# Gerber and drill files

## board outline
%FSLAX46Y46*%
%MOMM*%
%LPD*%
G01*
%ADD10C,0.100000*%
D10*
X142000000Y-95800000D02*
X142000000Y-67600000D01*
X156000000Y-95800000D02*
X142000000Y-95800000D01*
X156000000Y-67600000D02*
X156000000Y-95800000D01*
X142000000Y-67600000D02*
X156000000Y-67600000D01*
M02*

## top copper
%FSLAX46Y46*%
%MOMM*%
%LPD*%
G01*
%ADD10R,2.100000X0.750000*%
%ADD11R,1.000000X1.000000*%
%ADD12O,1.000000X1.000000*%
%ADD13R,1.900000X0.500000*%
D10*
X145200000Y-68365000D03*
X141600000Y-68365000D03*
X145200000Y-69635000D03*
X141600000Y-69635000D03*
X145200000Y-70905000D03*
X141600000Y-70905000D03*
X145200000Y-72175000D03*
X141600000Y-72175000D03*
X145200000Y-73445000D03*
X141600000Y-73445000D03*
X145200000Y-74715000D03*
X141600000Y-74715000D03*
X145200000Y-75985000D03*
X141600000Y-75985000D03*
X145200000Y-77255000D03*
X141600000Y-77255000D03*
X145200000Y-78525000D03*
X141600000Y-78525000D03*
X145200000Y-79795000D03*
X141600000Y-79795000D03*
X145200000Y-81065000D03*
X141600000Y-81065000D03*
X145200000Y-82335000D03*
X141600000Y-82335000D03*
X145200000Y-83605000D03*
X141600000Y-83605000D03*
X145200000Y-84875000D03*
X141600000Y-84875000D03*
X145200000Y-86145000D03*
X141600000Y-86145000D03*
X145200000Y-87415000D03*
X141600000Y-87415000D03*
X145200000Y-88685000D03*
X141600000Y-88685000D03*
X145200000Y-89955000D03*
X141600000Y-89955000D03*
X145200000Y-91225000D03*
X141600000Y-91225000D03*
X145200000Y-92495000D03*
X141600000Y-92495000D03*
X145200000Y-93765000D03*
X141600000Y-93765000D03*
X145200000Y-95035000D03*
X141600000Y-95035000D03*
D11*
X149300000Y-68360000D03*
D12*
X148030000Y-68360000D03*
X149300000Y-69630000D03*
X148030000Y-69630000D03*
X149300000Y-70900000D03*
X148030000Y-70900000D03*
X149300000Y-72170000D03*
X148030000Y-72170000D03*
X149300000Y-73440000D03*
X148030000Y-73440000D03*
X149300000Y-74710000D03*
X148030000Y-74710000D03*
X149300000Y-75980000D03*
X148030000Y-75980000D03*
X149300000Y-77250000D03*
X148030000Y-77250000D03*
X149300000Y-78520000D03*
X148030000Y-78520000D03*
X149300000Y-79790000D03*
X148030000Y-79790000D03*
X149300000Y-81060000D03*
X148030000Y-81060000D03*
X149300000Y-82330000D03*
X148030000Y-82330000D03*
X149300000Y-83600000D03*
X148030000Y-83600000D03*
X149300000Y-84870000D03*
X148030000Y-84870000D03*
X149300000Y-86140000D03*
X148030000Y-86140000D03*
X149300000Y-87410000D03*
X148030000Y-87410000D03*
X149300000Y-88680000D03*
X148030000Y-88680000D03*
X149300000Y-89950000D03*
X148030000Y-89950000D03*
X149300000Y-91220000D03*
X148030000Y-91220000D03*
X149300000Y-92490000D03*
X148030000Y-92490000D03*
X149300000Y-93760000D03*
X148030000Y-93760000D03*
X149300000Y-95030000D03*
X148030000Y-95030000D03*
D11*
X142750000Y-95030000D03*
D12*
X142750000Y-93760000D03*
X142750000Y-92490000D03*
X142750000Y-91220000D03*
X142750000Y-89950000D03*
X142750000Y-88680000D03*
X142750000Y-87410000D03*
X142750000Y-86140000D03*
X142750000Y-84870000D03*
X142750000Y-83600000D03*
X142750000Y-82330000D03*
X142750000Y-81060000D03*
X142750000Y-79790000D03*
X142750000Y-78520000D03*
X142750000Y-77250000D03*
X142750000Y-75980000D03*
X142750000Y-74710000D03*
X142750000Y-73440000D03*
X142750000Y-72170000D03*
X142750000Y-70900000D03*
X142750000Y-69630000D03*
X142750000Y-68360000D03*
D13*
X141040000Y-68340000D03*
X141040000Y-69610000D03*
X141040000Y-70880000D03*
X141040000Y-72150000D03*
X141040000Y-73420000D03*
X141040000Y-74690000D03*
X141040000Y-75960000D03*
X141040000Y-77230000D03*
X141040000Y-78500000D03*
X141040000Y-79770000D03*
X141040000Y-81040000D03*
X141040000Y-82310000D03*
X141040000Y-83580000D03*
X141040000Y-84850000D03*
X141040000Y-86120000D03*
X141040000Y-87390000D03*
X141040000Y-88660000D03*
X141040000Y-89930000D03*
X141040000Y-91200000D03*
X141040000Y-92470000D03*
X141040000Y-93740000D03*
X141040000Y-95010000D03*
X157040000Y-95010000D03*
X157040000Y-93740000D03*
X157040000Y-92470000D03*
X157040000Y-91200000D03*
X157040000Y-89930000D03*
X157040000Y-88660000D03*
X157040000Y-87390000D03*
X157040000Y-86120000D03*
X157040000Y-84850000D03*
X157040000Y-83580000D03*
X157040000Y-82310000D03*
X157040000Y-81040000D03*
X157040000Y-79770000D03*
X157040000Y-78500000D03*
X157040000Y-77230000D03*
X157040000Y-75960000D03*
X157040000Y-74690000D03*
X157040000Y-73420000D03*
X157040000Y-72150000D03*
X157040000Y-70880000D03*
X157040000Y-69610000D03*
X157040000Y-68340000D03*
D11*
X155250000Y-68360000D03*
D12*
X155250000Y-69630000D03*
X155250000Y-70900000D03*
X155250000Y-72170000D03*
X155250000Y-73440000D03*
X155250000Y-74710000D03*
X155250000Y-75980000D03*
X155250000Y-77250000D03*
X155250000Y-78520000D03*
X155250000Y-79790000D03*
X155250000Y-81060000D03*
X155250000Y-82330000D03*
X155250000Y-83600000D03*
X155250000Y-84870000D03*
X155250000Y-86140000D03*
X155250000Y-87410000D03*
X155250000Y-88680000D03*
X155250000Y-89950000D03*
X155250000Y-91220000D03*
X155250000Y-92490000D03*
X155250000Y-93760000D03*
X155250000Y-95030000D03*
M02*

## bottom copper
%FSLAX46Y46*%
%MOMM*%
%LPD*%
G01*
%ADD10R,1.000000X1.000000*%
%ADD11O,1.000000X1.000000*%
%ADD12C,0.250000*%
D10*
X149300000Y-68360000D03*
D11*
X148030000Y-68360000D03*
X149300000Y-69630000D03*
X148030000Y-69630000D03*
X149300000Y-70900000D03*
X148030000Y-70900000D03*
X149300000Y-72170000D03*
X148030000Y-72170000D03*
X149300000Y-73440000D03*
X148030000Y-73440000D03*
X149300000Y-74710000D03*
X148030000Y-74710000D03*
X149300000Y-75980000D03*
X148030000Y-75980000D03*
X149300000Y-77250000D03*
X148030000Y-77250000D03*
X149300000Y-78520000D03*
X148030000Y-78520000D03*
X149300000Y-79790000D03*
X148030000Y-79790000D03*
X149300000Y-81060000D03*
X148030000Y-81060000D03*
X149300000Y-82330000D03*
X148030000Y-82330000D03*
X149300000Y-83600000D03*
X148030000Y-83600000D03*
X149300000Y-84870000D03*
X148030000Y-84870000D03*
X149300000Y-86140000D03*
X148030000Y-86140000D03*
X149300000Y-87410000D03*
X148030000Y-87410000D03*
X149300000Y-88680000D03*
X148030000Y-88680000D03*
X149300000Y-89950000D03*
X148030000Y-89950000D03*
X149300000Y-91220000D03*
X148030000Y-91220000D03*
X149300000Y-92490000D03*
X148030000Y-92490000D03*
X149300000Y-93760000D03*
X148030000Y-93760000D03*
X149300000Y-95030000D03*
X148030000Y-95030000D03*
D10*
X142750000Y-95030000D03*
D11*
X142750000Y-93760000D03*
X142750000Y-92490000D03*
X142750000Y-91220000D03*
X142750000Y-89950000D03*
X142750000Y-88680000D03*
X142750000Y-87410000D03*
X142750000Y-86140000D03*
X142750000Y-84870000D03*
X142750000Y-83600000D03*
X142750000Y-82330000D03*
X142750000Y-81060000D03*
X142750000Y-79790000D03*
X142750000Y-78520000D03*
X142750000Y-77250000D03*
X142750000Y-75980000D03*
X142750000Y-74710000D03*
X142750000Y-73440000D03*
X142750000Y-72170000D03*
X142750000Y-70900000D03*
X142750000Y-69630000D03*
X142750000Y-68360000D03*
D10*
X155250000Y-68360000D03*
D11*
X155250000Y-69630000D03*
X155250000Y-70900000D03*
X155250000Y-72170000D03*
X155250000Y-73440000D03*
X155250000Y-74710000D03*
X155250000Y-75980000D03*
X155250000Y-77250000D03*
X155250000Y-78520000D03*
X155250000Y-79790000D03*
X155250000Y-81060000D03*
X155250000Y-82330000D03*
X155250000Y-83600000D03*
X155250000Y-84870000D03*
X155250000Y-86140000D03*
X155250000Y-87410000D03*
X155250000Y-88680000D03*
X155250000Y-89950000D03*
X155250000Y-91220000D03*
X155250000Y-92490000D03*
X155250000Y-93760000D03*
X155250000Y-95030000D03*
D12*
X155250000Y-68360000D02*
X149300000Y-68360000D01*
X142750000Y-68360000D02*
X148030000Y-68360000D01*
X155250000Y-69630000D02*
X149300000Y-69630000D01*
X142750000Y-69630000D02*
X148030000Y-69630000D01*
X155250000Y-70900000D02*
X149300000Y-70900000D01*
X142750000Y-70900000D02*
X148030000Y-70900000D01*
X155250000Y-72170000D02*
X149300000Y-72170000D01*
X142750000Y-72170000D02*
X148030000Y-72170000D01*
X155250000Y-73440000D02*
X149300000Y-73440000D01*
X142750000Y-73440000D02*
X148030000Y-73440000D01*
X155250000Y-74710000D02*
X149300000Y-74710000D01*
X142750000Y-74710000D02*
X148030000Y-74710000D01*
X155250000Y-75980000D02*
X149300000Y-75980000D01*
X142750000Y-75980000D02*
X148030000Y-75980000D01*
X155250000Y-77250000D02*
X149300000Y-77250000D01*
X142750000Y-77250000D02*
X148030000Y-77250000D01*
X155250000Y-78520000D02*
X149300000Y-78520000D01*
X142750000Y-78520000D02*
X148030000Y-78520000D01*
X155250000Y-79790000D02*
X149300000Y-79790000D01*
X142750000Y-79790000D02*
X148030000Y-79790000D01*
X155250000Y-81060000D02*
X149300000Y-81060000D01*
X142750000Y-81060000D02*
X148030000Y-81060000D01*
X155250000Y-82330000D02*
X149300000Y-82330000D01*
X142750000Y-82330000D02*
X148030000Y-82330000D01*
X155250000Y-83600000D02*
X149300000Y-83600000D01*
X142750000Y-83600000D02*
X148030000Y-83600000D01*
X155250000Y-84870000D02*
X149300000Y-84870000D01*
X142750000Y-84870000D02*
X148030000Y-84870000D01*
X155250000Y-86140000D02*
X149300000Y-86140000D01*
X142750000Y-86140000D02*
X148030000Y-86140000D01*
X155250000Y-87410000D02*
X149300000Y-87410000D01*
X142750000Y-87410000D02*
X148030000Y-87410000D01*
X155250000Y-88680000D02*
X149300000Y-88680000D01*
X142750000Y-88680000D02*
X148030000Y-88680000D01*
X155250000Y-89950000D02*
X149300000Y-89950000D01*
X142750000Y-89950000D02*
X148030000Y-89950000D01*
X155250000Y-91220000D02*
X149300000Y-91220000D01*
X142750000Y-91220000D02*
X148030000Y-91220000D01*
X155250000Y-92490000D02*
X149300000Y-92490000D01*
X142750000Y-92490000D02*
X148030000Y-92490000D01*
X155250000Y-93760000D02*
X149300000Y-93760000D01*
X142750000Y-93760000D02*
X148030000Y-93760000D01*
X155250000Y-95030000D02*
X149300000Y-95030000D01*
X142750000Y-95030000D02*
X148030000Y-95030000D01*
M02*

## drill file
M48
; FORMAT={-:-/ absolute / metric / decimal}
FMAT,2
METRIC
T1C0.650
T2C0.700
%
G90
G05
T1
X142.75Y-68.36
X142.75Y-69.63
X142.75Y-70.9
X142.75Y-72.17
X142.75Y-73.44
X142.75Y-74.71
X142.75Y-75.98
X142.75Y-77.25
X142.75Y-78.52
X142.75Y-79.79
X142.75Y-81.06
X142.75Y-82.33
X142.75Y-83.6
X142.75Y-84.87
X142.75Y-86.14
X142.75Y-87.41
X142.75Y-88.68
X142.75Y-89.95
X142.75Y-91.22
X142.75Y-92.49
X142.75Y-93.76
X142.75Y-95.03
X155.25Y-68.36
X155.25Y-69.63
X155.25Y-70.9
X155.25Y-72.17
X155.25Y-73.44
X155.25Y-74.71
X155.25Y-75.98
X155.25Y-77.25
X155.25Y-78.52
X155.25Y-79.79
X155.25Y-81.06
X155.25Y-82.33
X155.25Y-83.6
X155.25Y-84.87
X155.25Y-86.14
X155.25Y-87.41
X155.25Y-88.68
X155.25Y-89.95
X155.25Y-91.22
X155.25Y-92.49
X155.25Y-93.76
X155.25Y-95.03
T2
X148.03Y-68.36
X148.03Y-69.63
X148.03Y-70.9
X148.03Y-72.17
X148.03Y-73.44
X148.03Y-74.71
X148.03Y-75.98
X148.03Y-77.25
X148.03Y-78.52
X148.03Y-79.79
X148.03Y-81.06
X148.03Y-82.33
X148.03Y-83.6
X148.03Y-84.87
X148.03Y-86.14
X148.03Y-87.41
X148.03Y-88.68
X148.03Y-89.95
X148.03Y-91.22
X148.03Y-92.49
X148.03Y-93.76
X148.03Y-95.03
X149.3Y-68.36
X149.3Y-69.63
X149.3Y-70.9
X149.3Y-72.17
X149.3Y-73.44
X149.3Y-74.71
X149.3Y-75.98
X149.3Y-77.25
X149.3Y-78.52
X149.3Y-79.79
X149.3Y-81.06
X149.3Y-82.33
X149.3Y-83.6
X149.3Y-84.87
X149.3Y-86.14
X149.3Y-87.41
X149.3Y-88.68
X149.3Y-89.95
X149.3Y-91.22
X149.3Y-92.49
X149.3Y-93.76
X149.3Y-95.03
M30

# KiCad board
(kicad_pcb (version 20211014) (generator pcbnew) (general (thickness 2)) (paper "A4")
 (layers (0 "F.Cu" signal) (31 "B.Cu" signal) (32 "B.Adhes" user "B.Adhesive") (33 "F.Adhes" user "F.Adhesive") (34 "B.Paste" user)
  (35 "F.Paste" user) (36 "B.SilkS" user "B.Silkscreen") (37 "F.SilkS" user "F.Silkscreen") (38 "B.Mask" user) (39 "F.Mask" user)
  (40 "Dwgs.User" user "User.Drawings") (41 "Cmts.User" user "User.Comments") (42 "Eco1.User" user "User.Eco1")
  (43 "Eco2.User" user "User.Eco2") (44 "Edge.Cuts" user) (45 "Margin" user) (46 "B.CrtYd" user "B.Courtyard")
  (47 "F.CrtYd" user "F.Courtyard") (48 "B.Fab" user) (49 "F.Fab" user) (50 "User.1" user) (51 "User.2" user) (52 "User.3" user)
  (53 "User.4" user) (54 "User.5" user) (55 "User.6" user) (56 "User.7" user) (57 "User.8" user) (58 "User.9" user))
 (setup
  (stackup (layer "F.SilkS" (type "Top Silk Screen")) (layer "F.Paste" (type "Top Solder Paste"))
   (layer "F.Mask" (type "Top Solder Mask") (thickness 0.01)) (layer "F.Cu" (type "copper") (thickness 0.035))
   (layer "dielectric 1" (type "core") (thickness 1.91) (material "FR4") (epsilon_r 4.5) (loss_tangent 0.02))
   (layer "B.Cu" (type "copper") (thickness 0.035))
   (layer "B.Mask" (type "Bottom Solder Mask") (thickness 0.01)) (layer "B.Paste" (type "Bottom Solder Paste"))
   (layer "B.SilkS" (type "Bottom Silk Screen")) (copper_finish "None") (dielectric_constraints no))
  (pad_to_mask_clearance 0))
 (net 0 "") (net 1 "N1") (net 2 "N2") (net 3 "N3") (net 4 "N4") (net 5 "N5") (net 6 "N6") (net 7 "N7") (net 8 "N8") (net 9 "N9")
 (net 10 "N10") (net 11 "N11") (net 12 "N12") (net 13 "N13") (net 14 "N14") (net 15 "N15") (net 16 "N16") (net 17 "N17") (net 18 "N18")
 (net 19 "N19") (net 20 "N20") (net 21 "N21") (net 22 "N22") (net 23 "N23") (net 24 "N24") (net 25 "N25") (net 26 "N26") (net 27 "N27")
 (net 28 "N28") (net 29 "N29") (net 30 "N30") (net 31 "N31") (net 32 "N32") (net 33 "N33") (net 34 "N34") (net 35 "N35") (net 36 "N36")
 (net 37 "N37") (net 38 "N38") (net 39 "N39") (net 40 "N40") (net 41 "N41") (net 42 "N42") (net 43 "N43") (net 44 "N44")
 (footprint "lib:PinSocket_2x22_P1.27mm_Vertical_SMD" (layer "F.Cu") (at 143.4 81.7)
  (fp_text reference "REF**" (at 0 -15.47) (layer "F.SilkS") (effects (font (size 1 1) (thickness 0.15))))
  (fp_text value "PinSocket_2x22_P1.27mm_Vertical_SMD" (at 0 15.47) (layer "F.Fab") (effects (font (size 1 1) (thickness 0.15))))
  (pad "1" smd rect (at 1.8 -13.335) (size 2.1 0.75) (layers "F.Cu" "F.Paste" "F.Mask"))
  (pad "2" smd rect (at -1.8 -13.335) (size 2.1 0.75) (layers "F.Cu" "F.Paste" "F.Mask"))
  (pad "3" smd rect (at 1.8 -12.065) (size 2.1 0.75) (layers "F.Cu" "F.Paste" "F.Mask"))
  (pad "4" smd rect (at -1.8 -12.065) (size 2.1 0.75) (layers "F.Cu" "F.Paste" "F.Mask"))
  (pad "5" smd rect (at 1.8 -10.795) (size 2.1 0.75) (layers "F.Cu" "F.Paste" "F.Mask"))
  (pad "6" smd rect (at -1.8 -10.795) (size 2.1 0.75) (layers "F.Cu" "F.Paste" "F.Mask"))
  (pad "7" smd rect (at 1.8 -9.525) (size 2.1 0.75) (layers "F.Cu" "F.Paste" "F.Mask"))
  (pad "8" smd rect (at -1.8 -9.525) (size 2.1 0.75) (layers "F.Cu" "F.Paste" "F.Mask"))
  (pad "9" smd rect (at 1.8 -8.255) (size 2.1 0.75) (layers "F.Cu" "F.Paste" "F.Mask"))
  (pad "10" smd rect (at -1.8 -8.255) (size 2.1 0.75) (layers "F.Cu" "F.Paste" "F.Mask"))
  (pad "11" smd rect (at 1.8 -6.985) (size 2.1 0.75) (layers "F.Cu" "F.Paste" "F.Mask"))
  (pad "12" smd rect (at -1.8 -6.985) (size 2.1 0.75) (layers "F.Cu" "F.Paste" "F.Mask"))
  (pad "13" smd rect (at 1.8 -5.715) (size 2.1 0.75) (layers "F.Cu" "F.Paste" "F.Mask"))
  (pad "14" smd rect (at -1.8 -5.715) (size 2.1 0.75) (layers "F.Cu" "F.Paste" "F.Mask"))
  (pad "15" smd rect (at 1.8 -4.445) (size 2.1 0.75) (layers "F.Cu" "F.Paste" "F.Mask"))
  (pad "16" smd rect (at -1.8 -4.445) (size 2.1 0.75) (layers "F.Cu" "F.Paste" "F.Mask"))
  (pad "17" smd rect (at 1.8 -3.175) (size 2.1 0.75) (layers "F.Cu" "F.Paste" "F.Mask"))
  (pad "18" smd rect (at -1.8 -3.175) (size 2.1 0.75) (layers "F.Cu" "F.Paste" "F.Mask"))
  (pad "19" smd rect (at 1.8 -1.905) (size 2.1 0.75) (layers "F.Cu" "F.Paste" "F.Mask"))
  (pad "20" smd rect (at -1.8 -1.905) (size 2.1 0.75) (layers "F.Cu" "F.Paste" "F.Mask"))
  (pad "21" smd rect (at 1.8 -0.635) (size 2.1 0.75) (layers "F.Cu" "F.Paste" "F.Mask"))
  (pad "22" smd rect (at -1.8 -0.635) (size 2.1 0.75) (layers "F.Cu" "F.Paste" "F.Mask"))
  (pad "23" smd rect (at 1.8 0.635) (size 2.1 0.75) (layers "F.Cu" "F.Paste" "F.Mask"))
  (pad "24" smd rect (at -1.8 0.635) (size 2.1 0.75) (layers "F.Cu" "F.Paste" "F.Mask"))
  (pad "25" smd rect (at 1.8 1.905) (size 2.1 0.75) (layers "F.Cu" "F.Paste" "F.Mask"))
  (pad "26" smd rect (at -1.8 1.905) (size 2.1 0.75) (layers "F.Cu" "F.Paste" "F.Mask"))
  (pad "27" smd rect (at 1.8 3.175) (size 2.1 0.75) (layers "F.Cu" "F.Paste" "F.Mask"))
  (pad "28" smd rect (at -1.8 3.175) (size 2.1 0.75) (layers "F.Cu" "F.Paste" "F.Mask"))
  (pad "29" smd rect (at 1.8 4.445) (size 2.1 0.75) (layers "F.Cu" "F.Paste" "F.Mask"))
  (pad "30" smd rect (at -1.8 4.445) (size 2.1 0.75) (layers "F.Cu" "F.Paste" "F.Mask"))
  (pad "31" smd rect (at 1.8 5.715) (size 2.1 0.75) (layers "F.Cu" "F.Paste" "F.Mask"))
  (pad "32" smd rect (at -1.8 5.715) (size 2.1 0.75) (layers "F.Cu" "F.Paste" "F.Mask"))
  (pad "33" smd rect (at 1.8 6.985) (size 2.1 0.75) (layers "F.Cu" "F.Paste" "F.Mask"))
  (pad "34" smd rect (at -1.8 6.985) (size 2.1 0.75) (layers "F.Cu" "F.Paste" "F.Mask"))
  (pad "35" smd rect (at 1.8 8.255) (size 2.1 0.75) (layers "F.Cu" "F.Paste" "F.Mask"))
  (pad "36" smd rect (at -1.8 8.255) (size 2.1 0.75) (layers "F.Cu" "F.Paste" "F.Mask"))
  (pad "37" smd rect (at 1.8 9.525) (size 2.1 0.75) (layers "F.Cu" "F.Paste" "F.Mask"))
  (pad "38" smd rect (at -1.8 9.525) (size 2.1 0.75) (layers "F.Cu" "F.Paste" "F.Mask"))
  (pad "39" smd rect (at 1.8 10.795) (size 2.1 0.75) (layers "F.Cu" "F.Paste" "F.Mask"))
  (pad "40" smd rect (at -1.8 10.795) (size 2.1 0.75) (layers "F.Cu" "F.Paste" "F.Mask"))
  (pad "41" smd rect (at 1.8 12.065) (size 2.1 0.75) (layers "F.Cu" "F.Paste" "F.Mask"))
  (pad "42" smd rect (at -1.8 12.065) (size 2.1 0.75) (layers "F.Cu" "F.Paste" "F.Mask"))
  (pad "43" smd rect (at 1.8 13.335) (size 2.1 0.75) (layers "F.Cu" "F.Paste" "F.Mask"))
  (pad "44" smd rect (at -1.8 13.335) (size 2.1 0.75) (layers "F.Cu" "F.Paste" "F.Mask")))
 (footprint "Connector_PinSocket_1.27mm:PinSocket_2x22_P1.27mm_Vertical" (layer "F.Cu") (at 149.3 68.36)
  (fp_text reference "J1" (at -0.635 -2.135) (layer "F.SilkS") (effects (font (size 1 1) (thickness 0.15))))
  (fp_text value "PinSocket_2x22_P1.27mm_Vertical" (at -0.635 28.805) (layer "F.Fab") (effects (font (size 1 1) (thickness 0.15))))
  (pad "1" thru_hole rect (at 0 0) (size 1 1) (drill 0.7) (layers *.Cu *.Mask) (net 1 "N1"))
  (pad "2" thru_hole oval (at -1.27 0) (size 1 1) (drill 0.7) (layers *.Cu *.Mask) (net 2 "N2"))
  (pad "3" thru_hole oval (at 0 1.27) (size 1 1) (drill 0.7) (layers *.Cu *.Mask) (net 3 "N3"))
  (pad "4" thru_hole oval (at -1.27 1.27) (size 1 1) (drill 0.7) (layers *.Cu *.Mask) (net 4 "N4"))
  (pad "5" thru_hole oval (at 0 2.54) (size 1 1) (drill 0.7) (layers *.Cu *.Mask) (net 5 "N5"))
  (pad "6" thru_hole oval (at -1.27 2.54) (size 1 1) (drill 0.7) (layers *.Cu *.Mask) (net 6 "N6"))
  (pad "7" thru_hole oval (at 0 3.81) (size 1 1) (drill 0.7) (layers *.Cu *.Mask) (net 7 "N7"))
  (pad "8" thru_hole oval (at -1.27 3.81) (size 1 1) (drill 0.7) (layers *.Cu *.Mask) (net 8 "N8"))
  (pad "9" thru_hole oval (at 0 5.08) (size 1 1) (drill 0.7) (layers *.Cu *.Mask) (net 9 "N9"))
  (pad "10" thru_hole oval (at -1.27 5.08) (size 1 1) (drill 0.7) (layers *.Cu *.Mask) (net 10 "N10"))
  (pad "11" thru_hole oval (at 0 6.35) (size 1 1) (drill 0.7) (layers *.Cu *.Mask) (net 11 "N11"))
  (pad "12" thru_hole oval (at -1.27 6.35) (size 1 1) (drill 0.7) (layers *.Cu *.Mask) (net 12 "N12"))
  (pad "13" thru_hole oval (at 0 7.62) (size 1 1) (drill 0.7) (layers *.Cu *.Mask) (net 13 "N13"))
  (pad "14" thru_hole oval (at -1.27 7.62) (size 1 1) (drill 0.7) (layers *.Cu *.Mask) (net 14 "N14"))
  (pad "15" thru_hole oval (at 0 8.89) (size 1 1) (drill 0.7) (layers *.Cu *.Mask) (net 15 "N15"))
  (pad "16" thru_hole oval (at -1.27 8.89) (size 1 1) (drill 0.7) (layers *.Cu *.Mask) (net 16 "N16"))
  (pad "17" thru_hole oval (at 0 10.16) (size 1 1) (drill 0.7) (layers *.Cu *.Mask) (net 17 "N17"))
  (pad "18" thru_hole oval (at -1.27 10.16) (size 1 1) (drill 0.7) (layers *.Cu *.Mask) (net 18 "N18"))
  (pad "19" thru_hole oval (at 0 11.43) (size 1 1) (drill 0.7) (layers *.Cu *.Mask) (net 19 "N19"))
  (pad "20" thru_hole oval (at -1.27 11.43) (size 1 1) (drill 0.7) (layers *.Cu *.Mask) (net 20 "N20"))
  (pad "21" thru_hole oval (at 0 12.7) (size 1 1) (drill 0.7) (layers *.Cu *.Mask) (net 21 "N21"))
  (pad "22" thru_hole oval (at -1.27 12.7) (size 1 1) (drill 0.7) (layers *.Cu *.Mask) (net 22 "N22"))
  (pad "23" thru_hole oval (at 0 13.97) (size 1 1) (drill 0.7) (layers *.Cu *.Mask) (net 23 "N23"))
  (pad "24" thru_hole oval (at -1.27 13.97) (size 1 1) (drill 0.7) (layers *.Cu *.Mask) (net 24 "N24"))
  (pad "25" thru_hole oval (at 0 15.24) (size 1 1) (drill 0.7) (layers *.Cu *.Mask) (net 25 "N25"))
  (pad "26" thru_hole oval (at -1.27 15.24) (size 1 1) (drill 0.7) (layers *.Cu *.Mask) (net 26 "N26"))
  (pad "27" thru_hole oval (at 0 16.51) (size 1 1) (drill 0.7) (layers *.Cu *.Mask) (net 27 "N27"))
  (pad "28" thru_hole oval (at -1.27 16.51) (size 1 1) (drill 0.7) (layers *.Cu *.Mask) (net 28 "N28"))
  (pad "29" thru_hole oval (at 0 17.78) (size 1 1) (drill 0.7) (layers *.Cu *.Mask) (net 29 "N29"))
  (pad "30" thru_hole oval (at -1.27 17.78) (size 1 1) (drill 0.7) (layers *.Cu *.Mask) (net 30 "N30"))
  (pad "31" thru_hole oval (at 0 19.05) (size 1 1) (drill 0.7) (layers *.Cu *.Mask) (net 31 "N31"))
  (pad "32" thru_hole oval (at -1.27 19.05) (size 1 1) (drill 0.7) (layers *.Cu *.Mask) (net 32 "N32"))
  (pad "33" thru_hole oval (at 0 20.32) (size 1 1) (drill 0.7) (layers *.Cu *.Mask) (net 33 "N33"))
  (pad "34" thru_hole oval (at -1.27 20.32) (size 1 1) (drill 0.7) (layers *.Cu *.Mask) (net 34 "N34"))
  (pad "35" thru_hole oval (at 0 21.59) (size 1 1) (drill 0.7) (layers *.Cu *.Mask) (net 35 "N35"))
  (pad "36" thru_hole oval (at -1.27 21.59) (size 1 1) (drill 0.7) (layers *.Cu *.Mask) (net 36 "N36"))
  (pad "37" thru_hole oval (at 0 22.86) (size 1 1) (drill 0.7) (layers *.Cu *.Mask) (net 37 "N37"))
  (pad "38" thru_hole oval (at -1.27 22.86) (size 1 1) (drill 0.7) (layers *.Cu *.Mask) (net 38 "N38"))
  (pad "39" thru_hole oval (at 0 24.13) (size 1 1) (drill 0.7) (layers *.Cu *.Mask) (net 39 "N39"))
  (pad "40" thru_hole oval (at -1.27 24.13) (size 1 1) (drill 0.7) (layers *.Cu *.Mask) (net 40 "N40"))
  (pad "41" thru_hole oval (at 0 25.4) (size 1 1) (drill 0.7) (layers *.Cu *.Mask) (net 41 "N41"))
  (pad "42" thru_hole oval (at -1.27 25.4) (size 1 1) (drill 0.7) (layers *.Cu *.Mask) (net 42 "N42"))
  (pad "43" thru_hole oval (at 0 26.67) (size 1 1) (drill 0.7) (layers *.Cu *.Mask) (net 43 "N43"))
  (pad "44" thru_hole oval (at -1.27 26.67) (size 1 1) (drill 0.7) (layers *.Cu *.Mask) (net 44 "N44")))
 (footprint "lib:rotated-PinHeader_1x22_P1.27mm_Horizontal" (layer "F.Cu") (at 142.75 95.03 180)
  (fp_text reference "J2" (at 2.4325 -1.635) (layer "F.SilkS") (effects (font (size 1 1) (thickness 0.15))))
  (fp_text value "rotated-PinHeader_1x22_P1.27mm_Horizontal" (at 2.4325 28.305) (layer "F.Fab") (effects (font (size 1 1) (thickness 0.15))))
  (pad "1" thru_hole rect (at 0 0 180) (size 1 1) (drill 0.65) (layers *.Cu *.Mask) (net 44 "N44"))
  (pad "2" thru_hole oval (at 0 1.27 180) (size 1 1) (drill 0.65) (layers *.Cu *.Mask) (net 42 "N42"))
  (pad "3" thru_hole oval (at 0 2.54 180) (size 1 1) (drill 0.65) (layers *.Cu *.Mask) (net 40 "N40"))
  (pad "4" thru_hole oval (at 0 3.81 180) (size 1 1) (drill 0.65) (layers *.Cu *.Mask) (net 38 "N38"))
  (pad "5" thru_hole oval (at 0 5.08 180) (size 1 1) (drill 0.65) (layers *.Cu *.Mask) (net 36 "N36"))
  (pad "6" thru_hole oval (at 0 6.35 180) (size 1 1) (drill 0.65) (layers *.Cu *.Mask) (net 34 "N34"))
  (pad "7" thru_hole oval (at 0 7.62 180) (size 1 1) (drill 0.65) (layers *.Cu *.Mask) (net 32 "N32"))
  (pad "8" thru_hole oval (at 0 8.89 180) (size 1 1) (drill 0.65) (layers *.Cu *.Mask) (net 30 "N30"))
  (pad "9" thru_hole oval (at 0 10.16 180) (size 1 1) (drill 0.65) (layers *.Cu *.Mask) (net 28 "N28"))
  (pad "10" thru_hole oval (at 0 11.43 180) (size 1 1) (drill 0.65) (layers *.Cu *.Mask) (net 26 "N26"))
  (pad "11" thru_hole oval (at 0 12.7 180) (size 1 1) (drill 0.65) (layers *.Cu *.Mask) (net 24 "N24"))
  (pad "12" thru_hole oval (at 0 13.97 180) (size 1 1) (drill 0.65) (layers *.Cu *.Mask) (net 22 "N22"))
  (pad "13" thru_hole oval (at 0 15.24 180) (size 1 1) (drill 0.65) (layers *.Cu *.Mask) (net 20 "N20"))
  (pad "14" thru_hole oval (at 0 16.51 180) (size 1 1) (drill 0.65) (layers *.Cu *.Mask) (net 18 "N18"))
  (pad "15" thru_hole oval (at 0 17.78 180) (size 1 1) (drill 0.65) (layers *.Cu *.Mask) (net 16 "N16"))
  (pad "16" thru_hole oval (at 0 19.05 180) (size 1 1) (drill 0.65) (layers *.Cu *.Mask) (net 14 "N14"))
  (pad "17" thru_hole oval (at 0 20.32 180) (size 1 1) (drill 0.65) (layers *.Cu *.Mask) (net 12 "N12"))
  (pad "18" thru_hole oval (at 0 21.59 180) (size 1 1) (drill 0.65) (layers *.Cu *.Mask) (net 10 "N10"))
  (pad "19" thru_hole oval (at 0 22.86 180) (size 1 1) (drill 0.65) (layers *.Cu *.Mask) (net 8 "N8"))
  (pad "20" thru_hole oval (at 0 24.13 180) (size 1 1) (drill 0.65) (layers *.Cu *.Mask) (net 6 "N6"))
  (pad "21" thru_hole oval (at 0 25.4 180) (size 1 1) (drill 0.65) (layers *.Cu *.Mask) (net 4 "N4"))
  (pad "22" thru_hole oval (at 0 26.67 180) (size 1 1) (drill 0.65) (layers *.Cu *.Mask) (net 2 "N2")))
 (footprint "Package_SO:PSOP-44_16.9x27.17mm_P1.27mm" (layer "F.Cu") (at 149.04 81.675)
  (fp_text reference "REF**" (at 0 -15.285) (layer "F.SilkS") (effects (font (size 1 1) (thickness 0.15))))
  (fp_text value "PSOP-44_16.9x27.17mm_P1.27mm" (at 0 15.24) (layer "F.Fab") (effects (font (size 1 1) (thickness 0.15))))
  (pad "1" smd rect (at -8 -13.335 270) (size 0.5 1.9) (layers "F.Cu" "F.Paste" "F.Mask"))
  (pad "2" smd rect (at -8 -12.065 270) (size 0.5 1.9) (layers "F.Cu" "F.Paste" "F.Mask"))
  (pad "3" smd rect (at -8 -10.795 270) (size 0.5 1.9) (layers "F.Cu" "F.Paste" "F.Mask"))
  (pad "4" smd rect (at -8 -9.525 270) (size 0.5 1.9) (layers "F.Cu" "F.Paste" "F.Mask"))
  (pad "5" smd rect (at -8 -8.255 270) (size 0.5 1.9) (layers "F.Cu" "F.Paste" "F.Mask"))
  (pad "6" smd rect (at -8 -6.985 270) (size 0.5 1.9) (layers "F.Cu" "F.Paste" "F.Mask"))
  (pad "7" smd rect (at -8 -5.715 270) (size 0.5 1.9) (layers "F.Cu" "F.Paste" "F.Mask"))
  (pad "8" smd rect (at -8 -4.445 270) (size 0.5 1.9) (layers "F.Cu" "F.Paste" "F.Mask"))
  (pad "9" smd rect (at -8 -3.175 270) (size 0.5 1.9) (layers "F.Cu" "F.Paste" "F.Mask"))
  (pad "10" smd rect (at -8 -1.905 270) (size 0.5 1.9) (layers "F.Cu" "F.Paste" "F.Mask"))
  (pad "11" smd rect (at -8 -0.635 270) (size 0.5 1.9) (layers "F.Cu" "F.Paste" "F.Mask"))
  (pad "12" smd rect (at -8 0.635 270) (size 0.5 1.9) (layers "F.Cu" "F.Paste" "F.Mask"))
  (pad "13" smd rect (at -8 1.905 270) (size 0.5 1.9) (layers "F.Cu" "F.Paste" "F.Mask"))
  (pad "14" smd rect (at -8 3.175 270) (size 0.5 1.9) (layers "F.Cu" "F.Paste" "F.Mask"))
  (pad "15" smd rect (at -8 4.445 270) (size 0.5 1.9) (layers "F.Cu" "F.Paste" "F.Mask"))
  (pad "16" smd rect (at -8 5.715 270) (size 0.5 1.9) (layers "F.Cu" "F.Paste" "F.Mask"))
  (pad "17" smd rect (at -8 6.985 270) (size 0.5 1.9) (layers "F.Cu" "F.Paste" "F.Mask"))
  (pad "18" smd rect (at -8 8.255 270) (size 0.5 1.9) (layers "F.Cu" "F.Paste" "F.Mask"))
  (pad "19" smd rect (at -8 9.525 270) (size 0.5 1.9) (layers "F.Cu" "F.Paste" "F.Mask"))
  (pad "20" smd rect (at -8 10.795 270) (size 0.5 1.9) (layers "F.Cu" "F.Paste" "F.Mask"))
  (pad "21" smd rect (at -8 12.065 270) (size 0.5 1.9) (layers "F.Cu" "F.Paste" "F.Mask"))
  (pad "22" smd rect (at -8 13.335 270) (size 0.5 1.9) (layers "F.Cu" "F.Paste" "F.Mask"))
  (pad "23" smd rect (at 8 13.335 270) (size 0.5 1.9) (layers "F.Cu" "F.Paste" "F.Mask"))
  (pad "24" smd rect (at 8 12.065 270) (size 0.5 1.9) (layers "F.Cu" "F.Paste" "F.Mask"))
  (pad "25" smd rect (at 8 10.795 270) (size 0.5 1.9) (layers "F.Cu" "F.Paste" "F.Mask"))
  (pad "26" smd rect (at 8 9.525 270) (size 0.5 1.9) (layers "F.Cu" "F.Paste" "F.Mask"))
  (pad "27" smd rect (at 8 8.255 270) (size 0.5 1.9) (layers "F.Cu" "F.Paste" "F.Mask"))
  (pad "28" smd rect (at 8 6.985 270) (size 0.5 1.9) (layers "F.Cu" "F.Paste" "F.Mask"))
  (pad "29" smd rect (at 8 5.715 270) (size 0.5 1.9) (layers "F.Cu" "F.Paste" "F.Mask"))
  (pad "30" smd rect (at 8 4.445 270) (size 0.5 1.9) (layers "F.Cu" "F.Paste" "F.Mask"))
  (pad "31" smd rect (at 8 3.175 270) (size 0.5 1.9) (layers "F.Cu" "F.Paste" "F.Mask"))
  (pad "32" smd rect (at 8 1.905 270) (size 0.5 1.9) (layers "F.Cu" "F.Paste" "F.Mask"))
  (pad "33" smd rect (at 8 0.635 270) (size 0.5 1.9) (layers "F.Cu" "F.Paste" "F.Mask"))
  (pad "34" smd rect (at 8 -0.635 270) (size 0.5 1.9) (layers "F.Cu" "F.Paste" "F.Mask"))
  (pad "35" smd rect (at 8 -1.905 270) (size 0.5 1.9) (layers "F.Cu" "F.Paste" "F.Mask"))
  (pad "36" smd rect (at 8 -3.175 270) (size 0.5 1.9) (layers "F.Cu" "F.Paste" "F.Mask"))
  (pad "37" smd rect (at 8 -4.445 270) (size 0.5 1.9) (layers "F.Cu" "F.Paste" "F.Mask"))
  (pad "38" smd rect (at 8 -5.715 270) (size 0.5 1.9) (layers "F.Cu" "F.Paste" "F.Mask"))
  (pad "39" smd rect (at 8 -6.985 270) (size 0.5 1.9) (layers "F.Cu" "F.Paste" "F.Mask"))
  (pad "40" smd rect (at 8 -8.255 270) (size 0.5 1.9) (layers "F.Cu" "F.Paste" "F.Mask"))
  (pad "41" smd rect (at 8 -9.525 270) (size 0.5 1.9) (layers "F.Cu" "F.Paste" "F.Mask"))
  (pad "42" smd rect (at 8 -10.795 270) (size 0.5 1.9) (layers "F.Cu" "F.Paste" "F.Mask"))
  (pad "43" smd rect (at 8 -12.065 270) (size 0.5 1.9) (layers "F.Cu" "F.Paste" "F.Mask"))
  (pad "44" smd rect (at 8 -13.335 270) (size 0.5 1.9) (layers "F.Cu" "F.Paste" "F.Mask")))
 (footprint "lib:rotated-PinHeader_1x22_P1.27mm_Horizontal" (layer "F.Cu") (at 155.25 68.36)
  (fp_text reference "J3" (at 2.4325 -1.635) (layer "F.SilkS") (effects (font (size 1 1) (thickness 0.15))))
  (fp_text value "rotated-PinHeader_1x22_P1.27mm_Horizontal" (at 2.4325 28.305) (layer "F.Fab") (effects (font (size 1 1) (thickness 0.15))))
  (pad "1" thru_hole rect (at 0 0) (size 1 1) (drill 0.65) (layers *.Cu *.Mask) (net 1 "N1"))
  (pad "2" thru_hole oval (at 0 1.27) (size 1 1) (drill 0.65) (layers *.Cu *.Mask) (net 3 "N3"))
  (pad "3" thru_hole oval (at 0 2.54) (size 1 1) (drill 0.65) (layers *.Cu *.Mask) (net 5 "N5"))
  (pad "4" thru_hole oval (at 0 3.81) (size 1 1) (drill 0.65) (layers *.Cu *.Mask) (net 7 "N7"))
  (pad "5" thru_hole oval (at 0 5.08) (size 1 1) (drill 0.65) (layers *.Cu *.Mask) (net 9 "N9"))
  (pad "6" thru_hole oval (at 0 6.35) (size 1 1) (drill 0.65) (layers *.Cu *.Mask) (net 11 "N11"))
  (pad "7" thru_hole oval (at 0 7.62) (size 1 1) (drill 0.65) (layers *.Cu *.Mask) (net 13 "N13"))
  (pad "8" thru_hole oval (at 0 8.89) (size 1 1) (drill 0.65) (layers *.Cu *.Mask) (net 15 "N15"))
  (pad "9" thru_hole oval (at 0 10.16) (size 1 1) (drill 0.65) (layers *.Cu *.Mask) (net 17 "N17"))
  (pad "10" thru_hole oval (at 0 11.43) (size 1 1) (drill 0.65) (layers *.Cu *.Mask) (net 19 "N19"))
  (pad "11" thru_hole oval (at 0 12.7) (size 1 1) (drill 0.65) (layers *.Cu *.Mask) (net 21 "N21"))
  (pad "12" thru_hole oval (at 0 13.97) (size 1 1) (drill 0.65) (layers *.Cu *.Mask) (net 23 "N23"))
  (pad "13" thru_hole oval (at 0 15.24) (size 1 1) (drill 0.65) (layers *.Cu *.Mask) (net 25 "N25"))
  (pad "14" thru_hole oval (at 0 16.51) (size 1 1) (drill 0.65) (layers *.Cu *.Mask) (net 27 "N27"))
  (pad "15" thru_hole oval (at 0 17.78) (size 1 1) (drill 0.65) (layers *.Cu *.Mask) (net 29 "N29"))
  (pad "16" thru_hole oval (at 0 19.05) (size 1 1) (drill 0.65) (layers *.Cu *.Mask) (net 31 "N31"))
  (pad "17" thru_hole oval (at 0 20.32) (size 1 1) (drill 0.65) (layers *.Cu *.Mask) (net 33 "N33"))
  (pad "18" thru_hole oval (at 0 21.59) (size 1 1) (drill 0.65) (layers *.Cu *.Mask) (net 35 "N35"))
  (pad "19" thru_hole oval (at 0 22.86) (size 1 1) (drill 0.65) (layers *.Cu *.Mask) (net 37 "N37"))
  (pad "20" thru_hole oval (at 0 24.13) (size 1 1) (drill 0.65) (layers *.Cu *.Mask) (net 39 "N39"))
  (pad "21" thru_hole oval (at 0 25.4) (size 1 1) (drill 0.65) (layers *.Cu *.Mask) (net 41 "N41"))
  (pad "22" thru_hole oval (at 0 26.67) (size 1 1) (drill 0.65) (layers *.Cu *.Mask) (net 43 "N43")))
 (gr_line (start 142 95.8) (end 142 67.6) (layer "Edge.Cuts") (width 0.1))
 (gr_line (start 156 95.8) (end 142 95.8) (layer "Edge.Cuts") (width 0.1))
 (gr_line (start 156 67.6) (end 156 95.8) (layer "Edge.Cuts") (width 0.1))
 (gr_line (start 142 67.6) (end 156 67.6) (layer "Edge.Cuts") (width 0.1))
 (segment (start 155.25 68.36) (end 149.3 68.36) (width 0.25) (layer "B.Cu") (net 1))
 (segment (start 142.75 68.36) (end 148.03 68.36) (width 0.25) (layer "B.Cu") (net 2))
 (segment (start 155.25 69.63) (end 149.3 69.63) (width 0.25) (layer "B.Cu") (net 3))
 (segment (start 142.75 69.63) (end 148.03 69.63) (width 0.25) (layer "B.Cu") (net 4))
 (segment (start 155.25 70.9) (end 149.3 70.9) (width 0.25) (layer "B.Cu") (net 5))
 (segment (start 142.75 70.9) (end 148.03 70.9) (width 0.25) (layer "B.Cu") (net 6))
 (segment (start 155.25 72.17) (end 149.3 72.17) (width 0.25) (layer "B.Cu") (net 7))
 (segment (start 142.75 72.17) (end 148.03 72.17) (width 0.25) (layer "B.Cu") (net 8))
 (segment (start 155.25 73.44) (end 149.3 73.44) (width 0.25) (layer "B.Cu") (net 9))
 (segment (start 142.75 73.44) (end 148.03 73.44) (width 0.25) (layer "B.Cu") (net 10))
 (segment (start 155.25 74.71) (end 149.3 74.71) (width 0.25) (layer "B.Cu") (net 11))
 (segment (start 142.75 74.71) (end 148.03 74.71) (width 0.25) (layer "B.Cu") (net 12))
 (segment (start 155.25 75.98) (end 149.3 75.98) (width 0.25) (layer "B.Cu") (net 13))
 (segment (start 142.75 75.98) (end 148.03 75.98) (width 0.25) (layer "B.Cu") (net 14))
 (segment (start 155.25 77.25) (end 149.3 77.25) (width 0.25) (layer "B.Cu") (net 15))
 (segment (start 142.75 77.25) (end 148.03 77.25) (width 0.25) (layer "B.Cu") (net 16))
 (segment (start 155.25 78.52) (end 149.3 78.52) (width 0.25) (layer "B.Cu") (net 17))
 (segment (start 142.75 78.52) (end 148.03 78.52) (width 0.25) (layer "B.Cu") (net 18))
 (segment (start 155.25 79.79) (end 149.3 79.79) (width 0.25) (layer "B.Cu") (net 19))
 (segment (start 142.75 79.79) (end 148.03 79.79) (width 0.25) (layer "B.Cu") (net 20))
 (segment (start 155.25 81.06) (end 149.3 81.06) (width 0.25) (layer "B.Cu") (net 21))
 (segment (start 142.75 81.06) (end 148.03 81.06) (width 0.25) (layer "B.Cu") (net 22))
 (segment (start 155.25 82.33) (end 149.3 82.33) (width 0.25) (layer "B.Cu") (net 23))
 (segment (start 142.75 82.33) (end 148.03 82.33) (width 0.25) (layer "B.Cu") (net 24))
 (segment (start 155.25 83.6) (end 149.3 83.6) (width 0.25) (layer "B.Cu") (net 25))
 (segment (start 142.75 83.6) (end 148.03 83.6) (width 0.25) (layer "B.Cu") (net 26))
 (segment (start 155.25 84.87) (end 149.3 84.87) (width 0.25) (layer "B.Cu") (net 27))
 (segment (start 142.75 84.87) (end 148.03 84.87) (width 0.25) (layer "B.Cu") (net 28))
 (segment (start 155.25 86.14) (end 149.3 86.14) (width 0.25) (layer "B.Cu") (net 29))
 (segment (start 142.75 86.14) (end 148.03 86.14) (width 0.25) (layer "B.Cu") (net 30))
 (segment (start 155.25 87.41) (end 149.3 87.41) (width 0.25) (layer "B.Cu") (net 31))
 (segment (start 142.75 87.41) (end 148.03 87.41) (width 0.25) (layer "B.Cu") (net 32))
 (segment (start 155.25 88.68) (end 149.3 88.68) (width 0.25) (layer "B.Cu") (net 33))
 (segment (start 142.75 88.68) (end 148.03 88.68) (width 0.25) (layer "B.Cu") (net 34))
 (segment (start 155.25 89.95) (end 149.3 89.95) (width 0.25) (layer "B.Cu") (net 35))
 (segment (start 142.75 89.95) (end 148.03 89.95) (width 0.25) (layer "B.Cu") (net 36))
 (segment (start 155.25 91.22) (end 149.3 91.22) (width 0.25) (layer "B.Cu") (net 37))
 (segment (start 142.75 91.22) (end 148.03 91.22) (width 0.25) (layer "B.Cu") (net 38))
 (segment (start 155.25 92.49) (end 149.3 92.49) (width 0.25) (layer "B.Cu") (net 39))
 (segment (start 142.75 92.49) (end 148.03 92.49) (width 0.25) (layer "B.Cu") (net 40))
 (segment (start 155.25 93.76) (end 149.3 93.76) (width 0.25) (layer "B.Cu") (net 41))
 (segment (start 142.75 93.76) (end 148.03 93.76) (width 0.25) (layer "B.Cu") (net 42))
 (segment (start 155.25 95.03) (end 149.3 95.03) (width 0.25) (layer "B.Cu") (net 43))
 (segment (start 142.75 95.03) (end 148.03 95.03) (width 0.25) (layer "B.Cu") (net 44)))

